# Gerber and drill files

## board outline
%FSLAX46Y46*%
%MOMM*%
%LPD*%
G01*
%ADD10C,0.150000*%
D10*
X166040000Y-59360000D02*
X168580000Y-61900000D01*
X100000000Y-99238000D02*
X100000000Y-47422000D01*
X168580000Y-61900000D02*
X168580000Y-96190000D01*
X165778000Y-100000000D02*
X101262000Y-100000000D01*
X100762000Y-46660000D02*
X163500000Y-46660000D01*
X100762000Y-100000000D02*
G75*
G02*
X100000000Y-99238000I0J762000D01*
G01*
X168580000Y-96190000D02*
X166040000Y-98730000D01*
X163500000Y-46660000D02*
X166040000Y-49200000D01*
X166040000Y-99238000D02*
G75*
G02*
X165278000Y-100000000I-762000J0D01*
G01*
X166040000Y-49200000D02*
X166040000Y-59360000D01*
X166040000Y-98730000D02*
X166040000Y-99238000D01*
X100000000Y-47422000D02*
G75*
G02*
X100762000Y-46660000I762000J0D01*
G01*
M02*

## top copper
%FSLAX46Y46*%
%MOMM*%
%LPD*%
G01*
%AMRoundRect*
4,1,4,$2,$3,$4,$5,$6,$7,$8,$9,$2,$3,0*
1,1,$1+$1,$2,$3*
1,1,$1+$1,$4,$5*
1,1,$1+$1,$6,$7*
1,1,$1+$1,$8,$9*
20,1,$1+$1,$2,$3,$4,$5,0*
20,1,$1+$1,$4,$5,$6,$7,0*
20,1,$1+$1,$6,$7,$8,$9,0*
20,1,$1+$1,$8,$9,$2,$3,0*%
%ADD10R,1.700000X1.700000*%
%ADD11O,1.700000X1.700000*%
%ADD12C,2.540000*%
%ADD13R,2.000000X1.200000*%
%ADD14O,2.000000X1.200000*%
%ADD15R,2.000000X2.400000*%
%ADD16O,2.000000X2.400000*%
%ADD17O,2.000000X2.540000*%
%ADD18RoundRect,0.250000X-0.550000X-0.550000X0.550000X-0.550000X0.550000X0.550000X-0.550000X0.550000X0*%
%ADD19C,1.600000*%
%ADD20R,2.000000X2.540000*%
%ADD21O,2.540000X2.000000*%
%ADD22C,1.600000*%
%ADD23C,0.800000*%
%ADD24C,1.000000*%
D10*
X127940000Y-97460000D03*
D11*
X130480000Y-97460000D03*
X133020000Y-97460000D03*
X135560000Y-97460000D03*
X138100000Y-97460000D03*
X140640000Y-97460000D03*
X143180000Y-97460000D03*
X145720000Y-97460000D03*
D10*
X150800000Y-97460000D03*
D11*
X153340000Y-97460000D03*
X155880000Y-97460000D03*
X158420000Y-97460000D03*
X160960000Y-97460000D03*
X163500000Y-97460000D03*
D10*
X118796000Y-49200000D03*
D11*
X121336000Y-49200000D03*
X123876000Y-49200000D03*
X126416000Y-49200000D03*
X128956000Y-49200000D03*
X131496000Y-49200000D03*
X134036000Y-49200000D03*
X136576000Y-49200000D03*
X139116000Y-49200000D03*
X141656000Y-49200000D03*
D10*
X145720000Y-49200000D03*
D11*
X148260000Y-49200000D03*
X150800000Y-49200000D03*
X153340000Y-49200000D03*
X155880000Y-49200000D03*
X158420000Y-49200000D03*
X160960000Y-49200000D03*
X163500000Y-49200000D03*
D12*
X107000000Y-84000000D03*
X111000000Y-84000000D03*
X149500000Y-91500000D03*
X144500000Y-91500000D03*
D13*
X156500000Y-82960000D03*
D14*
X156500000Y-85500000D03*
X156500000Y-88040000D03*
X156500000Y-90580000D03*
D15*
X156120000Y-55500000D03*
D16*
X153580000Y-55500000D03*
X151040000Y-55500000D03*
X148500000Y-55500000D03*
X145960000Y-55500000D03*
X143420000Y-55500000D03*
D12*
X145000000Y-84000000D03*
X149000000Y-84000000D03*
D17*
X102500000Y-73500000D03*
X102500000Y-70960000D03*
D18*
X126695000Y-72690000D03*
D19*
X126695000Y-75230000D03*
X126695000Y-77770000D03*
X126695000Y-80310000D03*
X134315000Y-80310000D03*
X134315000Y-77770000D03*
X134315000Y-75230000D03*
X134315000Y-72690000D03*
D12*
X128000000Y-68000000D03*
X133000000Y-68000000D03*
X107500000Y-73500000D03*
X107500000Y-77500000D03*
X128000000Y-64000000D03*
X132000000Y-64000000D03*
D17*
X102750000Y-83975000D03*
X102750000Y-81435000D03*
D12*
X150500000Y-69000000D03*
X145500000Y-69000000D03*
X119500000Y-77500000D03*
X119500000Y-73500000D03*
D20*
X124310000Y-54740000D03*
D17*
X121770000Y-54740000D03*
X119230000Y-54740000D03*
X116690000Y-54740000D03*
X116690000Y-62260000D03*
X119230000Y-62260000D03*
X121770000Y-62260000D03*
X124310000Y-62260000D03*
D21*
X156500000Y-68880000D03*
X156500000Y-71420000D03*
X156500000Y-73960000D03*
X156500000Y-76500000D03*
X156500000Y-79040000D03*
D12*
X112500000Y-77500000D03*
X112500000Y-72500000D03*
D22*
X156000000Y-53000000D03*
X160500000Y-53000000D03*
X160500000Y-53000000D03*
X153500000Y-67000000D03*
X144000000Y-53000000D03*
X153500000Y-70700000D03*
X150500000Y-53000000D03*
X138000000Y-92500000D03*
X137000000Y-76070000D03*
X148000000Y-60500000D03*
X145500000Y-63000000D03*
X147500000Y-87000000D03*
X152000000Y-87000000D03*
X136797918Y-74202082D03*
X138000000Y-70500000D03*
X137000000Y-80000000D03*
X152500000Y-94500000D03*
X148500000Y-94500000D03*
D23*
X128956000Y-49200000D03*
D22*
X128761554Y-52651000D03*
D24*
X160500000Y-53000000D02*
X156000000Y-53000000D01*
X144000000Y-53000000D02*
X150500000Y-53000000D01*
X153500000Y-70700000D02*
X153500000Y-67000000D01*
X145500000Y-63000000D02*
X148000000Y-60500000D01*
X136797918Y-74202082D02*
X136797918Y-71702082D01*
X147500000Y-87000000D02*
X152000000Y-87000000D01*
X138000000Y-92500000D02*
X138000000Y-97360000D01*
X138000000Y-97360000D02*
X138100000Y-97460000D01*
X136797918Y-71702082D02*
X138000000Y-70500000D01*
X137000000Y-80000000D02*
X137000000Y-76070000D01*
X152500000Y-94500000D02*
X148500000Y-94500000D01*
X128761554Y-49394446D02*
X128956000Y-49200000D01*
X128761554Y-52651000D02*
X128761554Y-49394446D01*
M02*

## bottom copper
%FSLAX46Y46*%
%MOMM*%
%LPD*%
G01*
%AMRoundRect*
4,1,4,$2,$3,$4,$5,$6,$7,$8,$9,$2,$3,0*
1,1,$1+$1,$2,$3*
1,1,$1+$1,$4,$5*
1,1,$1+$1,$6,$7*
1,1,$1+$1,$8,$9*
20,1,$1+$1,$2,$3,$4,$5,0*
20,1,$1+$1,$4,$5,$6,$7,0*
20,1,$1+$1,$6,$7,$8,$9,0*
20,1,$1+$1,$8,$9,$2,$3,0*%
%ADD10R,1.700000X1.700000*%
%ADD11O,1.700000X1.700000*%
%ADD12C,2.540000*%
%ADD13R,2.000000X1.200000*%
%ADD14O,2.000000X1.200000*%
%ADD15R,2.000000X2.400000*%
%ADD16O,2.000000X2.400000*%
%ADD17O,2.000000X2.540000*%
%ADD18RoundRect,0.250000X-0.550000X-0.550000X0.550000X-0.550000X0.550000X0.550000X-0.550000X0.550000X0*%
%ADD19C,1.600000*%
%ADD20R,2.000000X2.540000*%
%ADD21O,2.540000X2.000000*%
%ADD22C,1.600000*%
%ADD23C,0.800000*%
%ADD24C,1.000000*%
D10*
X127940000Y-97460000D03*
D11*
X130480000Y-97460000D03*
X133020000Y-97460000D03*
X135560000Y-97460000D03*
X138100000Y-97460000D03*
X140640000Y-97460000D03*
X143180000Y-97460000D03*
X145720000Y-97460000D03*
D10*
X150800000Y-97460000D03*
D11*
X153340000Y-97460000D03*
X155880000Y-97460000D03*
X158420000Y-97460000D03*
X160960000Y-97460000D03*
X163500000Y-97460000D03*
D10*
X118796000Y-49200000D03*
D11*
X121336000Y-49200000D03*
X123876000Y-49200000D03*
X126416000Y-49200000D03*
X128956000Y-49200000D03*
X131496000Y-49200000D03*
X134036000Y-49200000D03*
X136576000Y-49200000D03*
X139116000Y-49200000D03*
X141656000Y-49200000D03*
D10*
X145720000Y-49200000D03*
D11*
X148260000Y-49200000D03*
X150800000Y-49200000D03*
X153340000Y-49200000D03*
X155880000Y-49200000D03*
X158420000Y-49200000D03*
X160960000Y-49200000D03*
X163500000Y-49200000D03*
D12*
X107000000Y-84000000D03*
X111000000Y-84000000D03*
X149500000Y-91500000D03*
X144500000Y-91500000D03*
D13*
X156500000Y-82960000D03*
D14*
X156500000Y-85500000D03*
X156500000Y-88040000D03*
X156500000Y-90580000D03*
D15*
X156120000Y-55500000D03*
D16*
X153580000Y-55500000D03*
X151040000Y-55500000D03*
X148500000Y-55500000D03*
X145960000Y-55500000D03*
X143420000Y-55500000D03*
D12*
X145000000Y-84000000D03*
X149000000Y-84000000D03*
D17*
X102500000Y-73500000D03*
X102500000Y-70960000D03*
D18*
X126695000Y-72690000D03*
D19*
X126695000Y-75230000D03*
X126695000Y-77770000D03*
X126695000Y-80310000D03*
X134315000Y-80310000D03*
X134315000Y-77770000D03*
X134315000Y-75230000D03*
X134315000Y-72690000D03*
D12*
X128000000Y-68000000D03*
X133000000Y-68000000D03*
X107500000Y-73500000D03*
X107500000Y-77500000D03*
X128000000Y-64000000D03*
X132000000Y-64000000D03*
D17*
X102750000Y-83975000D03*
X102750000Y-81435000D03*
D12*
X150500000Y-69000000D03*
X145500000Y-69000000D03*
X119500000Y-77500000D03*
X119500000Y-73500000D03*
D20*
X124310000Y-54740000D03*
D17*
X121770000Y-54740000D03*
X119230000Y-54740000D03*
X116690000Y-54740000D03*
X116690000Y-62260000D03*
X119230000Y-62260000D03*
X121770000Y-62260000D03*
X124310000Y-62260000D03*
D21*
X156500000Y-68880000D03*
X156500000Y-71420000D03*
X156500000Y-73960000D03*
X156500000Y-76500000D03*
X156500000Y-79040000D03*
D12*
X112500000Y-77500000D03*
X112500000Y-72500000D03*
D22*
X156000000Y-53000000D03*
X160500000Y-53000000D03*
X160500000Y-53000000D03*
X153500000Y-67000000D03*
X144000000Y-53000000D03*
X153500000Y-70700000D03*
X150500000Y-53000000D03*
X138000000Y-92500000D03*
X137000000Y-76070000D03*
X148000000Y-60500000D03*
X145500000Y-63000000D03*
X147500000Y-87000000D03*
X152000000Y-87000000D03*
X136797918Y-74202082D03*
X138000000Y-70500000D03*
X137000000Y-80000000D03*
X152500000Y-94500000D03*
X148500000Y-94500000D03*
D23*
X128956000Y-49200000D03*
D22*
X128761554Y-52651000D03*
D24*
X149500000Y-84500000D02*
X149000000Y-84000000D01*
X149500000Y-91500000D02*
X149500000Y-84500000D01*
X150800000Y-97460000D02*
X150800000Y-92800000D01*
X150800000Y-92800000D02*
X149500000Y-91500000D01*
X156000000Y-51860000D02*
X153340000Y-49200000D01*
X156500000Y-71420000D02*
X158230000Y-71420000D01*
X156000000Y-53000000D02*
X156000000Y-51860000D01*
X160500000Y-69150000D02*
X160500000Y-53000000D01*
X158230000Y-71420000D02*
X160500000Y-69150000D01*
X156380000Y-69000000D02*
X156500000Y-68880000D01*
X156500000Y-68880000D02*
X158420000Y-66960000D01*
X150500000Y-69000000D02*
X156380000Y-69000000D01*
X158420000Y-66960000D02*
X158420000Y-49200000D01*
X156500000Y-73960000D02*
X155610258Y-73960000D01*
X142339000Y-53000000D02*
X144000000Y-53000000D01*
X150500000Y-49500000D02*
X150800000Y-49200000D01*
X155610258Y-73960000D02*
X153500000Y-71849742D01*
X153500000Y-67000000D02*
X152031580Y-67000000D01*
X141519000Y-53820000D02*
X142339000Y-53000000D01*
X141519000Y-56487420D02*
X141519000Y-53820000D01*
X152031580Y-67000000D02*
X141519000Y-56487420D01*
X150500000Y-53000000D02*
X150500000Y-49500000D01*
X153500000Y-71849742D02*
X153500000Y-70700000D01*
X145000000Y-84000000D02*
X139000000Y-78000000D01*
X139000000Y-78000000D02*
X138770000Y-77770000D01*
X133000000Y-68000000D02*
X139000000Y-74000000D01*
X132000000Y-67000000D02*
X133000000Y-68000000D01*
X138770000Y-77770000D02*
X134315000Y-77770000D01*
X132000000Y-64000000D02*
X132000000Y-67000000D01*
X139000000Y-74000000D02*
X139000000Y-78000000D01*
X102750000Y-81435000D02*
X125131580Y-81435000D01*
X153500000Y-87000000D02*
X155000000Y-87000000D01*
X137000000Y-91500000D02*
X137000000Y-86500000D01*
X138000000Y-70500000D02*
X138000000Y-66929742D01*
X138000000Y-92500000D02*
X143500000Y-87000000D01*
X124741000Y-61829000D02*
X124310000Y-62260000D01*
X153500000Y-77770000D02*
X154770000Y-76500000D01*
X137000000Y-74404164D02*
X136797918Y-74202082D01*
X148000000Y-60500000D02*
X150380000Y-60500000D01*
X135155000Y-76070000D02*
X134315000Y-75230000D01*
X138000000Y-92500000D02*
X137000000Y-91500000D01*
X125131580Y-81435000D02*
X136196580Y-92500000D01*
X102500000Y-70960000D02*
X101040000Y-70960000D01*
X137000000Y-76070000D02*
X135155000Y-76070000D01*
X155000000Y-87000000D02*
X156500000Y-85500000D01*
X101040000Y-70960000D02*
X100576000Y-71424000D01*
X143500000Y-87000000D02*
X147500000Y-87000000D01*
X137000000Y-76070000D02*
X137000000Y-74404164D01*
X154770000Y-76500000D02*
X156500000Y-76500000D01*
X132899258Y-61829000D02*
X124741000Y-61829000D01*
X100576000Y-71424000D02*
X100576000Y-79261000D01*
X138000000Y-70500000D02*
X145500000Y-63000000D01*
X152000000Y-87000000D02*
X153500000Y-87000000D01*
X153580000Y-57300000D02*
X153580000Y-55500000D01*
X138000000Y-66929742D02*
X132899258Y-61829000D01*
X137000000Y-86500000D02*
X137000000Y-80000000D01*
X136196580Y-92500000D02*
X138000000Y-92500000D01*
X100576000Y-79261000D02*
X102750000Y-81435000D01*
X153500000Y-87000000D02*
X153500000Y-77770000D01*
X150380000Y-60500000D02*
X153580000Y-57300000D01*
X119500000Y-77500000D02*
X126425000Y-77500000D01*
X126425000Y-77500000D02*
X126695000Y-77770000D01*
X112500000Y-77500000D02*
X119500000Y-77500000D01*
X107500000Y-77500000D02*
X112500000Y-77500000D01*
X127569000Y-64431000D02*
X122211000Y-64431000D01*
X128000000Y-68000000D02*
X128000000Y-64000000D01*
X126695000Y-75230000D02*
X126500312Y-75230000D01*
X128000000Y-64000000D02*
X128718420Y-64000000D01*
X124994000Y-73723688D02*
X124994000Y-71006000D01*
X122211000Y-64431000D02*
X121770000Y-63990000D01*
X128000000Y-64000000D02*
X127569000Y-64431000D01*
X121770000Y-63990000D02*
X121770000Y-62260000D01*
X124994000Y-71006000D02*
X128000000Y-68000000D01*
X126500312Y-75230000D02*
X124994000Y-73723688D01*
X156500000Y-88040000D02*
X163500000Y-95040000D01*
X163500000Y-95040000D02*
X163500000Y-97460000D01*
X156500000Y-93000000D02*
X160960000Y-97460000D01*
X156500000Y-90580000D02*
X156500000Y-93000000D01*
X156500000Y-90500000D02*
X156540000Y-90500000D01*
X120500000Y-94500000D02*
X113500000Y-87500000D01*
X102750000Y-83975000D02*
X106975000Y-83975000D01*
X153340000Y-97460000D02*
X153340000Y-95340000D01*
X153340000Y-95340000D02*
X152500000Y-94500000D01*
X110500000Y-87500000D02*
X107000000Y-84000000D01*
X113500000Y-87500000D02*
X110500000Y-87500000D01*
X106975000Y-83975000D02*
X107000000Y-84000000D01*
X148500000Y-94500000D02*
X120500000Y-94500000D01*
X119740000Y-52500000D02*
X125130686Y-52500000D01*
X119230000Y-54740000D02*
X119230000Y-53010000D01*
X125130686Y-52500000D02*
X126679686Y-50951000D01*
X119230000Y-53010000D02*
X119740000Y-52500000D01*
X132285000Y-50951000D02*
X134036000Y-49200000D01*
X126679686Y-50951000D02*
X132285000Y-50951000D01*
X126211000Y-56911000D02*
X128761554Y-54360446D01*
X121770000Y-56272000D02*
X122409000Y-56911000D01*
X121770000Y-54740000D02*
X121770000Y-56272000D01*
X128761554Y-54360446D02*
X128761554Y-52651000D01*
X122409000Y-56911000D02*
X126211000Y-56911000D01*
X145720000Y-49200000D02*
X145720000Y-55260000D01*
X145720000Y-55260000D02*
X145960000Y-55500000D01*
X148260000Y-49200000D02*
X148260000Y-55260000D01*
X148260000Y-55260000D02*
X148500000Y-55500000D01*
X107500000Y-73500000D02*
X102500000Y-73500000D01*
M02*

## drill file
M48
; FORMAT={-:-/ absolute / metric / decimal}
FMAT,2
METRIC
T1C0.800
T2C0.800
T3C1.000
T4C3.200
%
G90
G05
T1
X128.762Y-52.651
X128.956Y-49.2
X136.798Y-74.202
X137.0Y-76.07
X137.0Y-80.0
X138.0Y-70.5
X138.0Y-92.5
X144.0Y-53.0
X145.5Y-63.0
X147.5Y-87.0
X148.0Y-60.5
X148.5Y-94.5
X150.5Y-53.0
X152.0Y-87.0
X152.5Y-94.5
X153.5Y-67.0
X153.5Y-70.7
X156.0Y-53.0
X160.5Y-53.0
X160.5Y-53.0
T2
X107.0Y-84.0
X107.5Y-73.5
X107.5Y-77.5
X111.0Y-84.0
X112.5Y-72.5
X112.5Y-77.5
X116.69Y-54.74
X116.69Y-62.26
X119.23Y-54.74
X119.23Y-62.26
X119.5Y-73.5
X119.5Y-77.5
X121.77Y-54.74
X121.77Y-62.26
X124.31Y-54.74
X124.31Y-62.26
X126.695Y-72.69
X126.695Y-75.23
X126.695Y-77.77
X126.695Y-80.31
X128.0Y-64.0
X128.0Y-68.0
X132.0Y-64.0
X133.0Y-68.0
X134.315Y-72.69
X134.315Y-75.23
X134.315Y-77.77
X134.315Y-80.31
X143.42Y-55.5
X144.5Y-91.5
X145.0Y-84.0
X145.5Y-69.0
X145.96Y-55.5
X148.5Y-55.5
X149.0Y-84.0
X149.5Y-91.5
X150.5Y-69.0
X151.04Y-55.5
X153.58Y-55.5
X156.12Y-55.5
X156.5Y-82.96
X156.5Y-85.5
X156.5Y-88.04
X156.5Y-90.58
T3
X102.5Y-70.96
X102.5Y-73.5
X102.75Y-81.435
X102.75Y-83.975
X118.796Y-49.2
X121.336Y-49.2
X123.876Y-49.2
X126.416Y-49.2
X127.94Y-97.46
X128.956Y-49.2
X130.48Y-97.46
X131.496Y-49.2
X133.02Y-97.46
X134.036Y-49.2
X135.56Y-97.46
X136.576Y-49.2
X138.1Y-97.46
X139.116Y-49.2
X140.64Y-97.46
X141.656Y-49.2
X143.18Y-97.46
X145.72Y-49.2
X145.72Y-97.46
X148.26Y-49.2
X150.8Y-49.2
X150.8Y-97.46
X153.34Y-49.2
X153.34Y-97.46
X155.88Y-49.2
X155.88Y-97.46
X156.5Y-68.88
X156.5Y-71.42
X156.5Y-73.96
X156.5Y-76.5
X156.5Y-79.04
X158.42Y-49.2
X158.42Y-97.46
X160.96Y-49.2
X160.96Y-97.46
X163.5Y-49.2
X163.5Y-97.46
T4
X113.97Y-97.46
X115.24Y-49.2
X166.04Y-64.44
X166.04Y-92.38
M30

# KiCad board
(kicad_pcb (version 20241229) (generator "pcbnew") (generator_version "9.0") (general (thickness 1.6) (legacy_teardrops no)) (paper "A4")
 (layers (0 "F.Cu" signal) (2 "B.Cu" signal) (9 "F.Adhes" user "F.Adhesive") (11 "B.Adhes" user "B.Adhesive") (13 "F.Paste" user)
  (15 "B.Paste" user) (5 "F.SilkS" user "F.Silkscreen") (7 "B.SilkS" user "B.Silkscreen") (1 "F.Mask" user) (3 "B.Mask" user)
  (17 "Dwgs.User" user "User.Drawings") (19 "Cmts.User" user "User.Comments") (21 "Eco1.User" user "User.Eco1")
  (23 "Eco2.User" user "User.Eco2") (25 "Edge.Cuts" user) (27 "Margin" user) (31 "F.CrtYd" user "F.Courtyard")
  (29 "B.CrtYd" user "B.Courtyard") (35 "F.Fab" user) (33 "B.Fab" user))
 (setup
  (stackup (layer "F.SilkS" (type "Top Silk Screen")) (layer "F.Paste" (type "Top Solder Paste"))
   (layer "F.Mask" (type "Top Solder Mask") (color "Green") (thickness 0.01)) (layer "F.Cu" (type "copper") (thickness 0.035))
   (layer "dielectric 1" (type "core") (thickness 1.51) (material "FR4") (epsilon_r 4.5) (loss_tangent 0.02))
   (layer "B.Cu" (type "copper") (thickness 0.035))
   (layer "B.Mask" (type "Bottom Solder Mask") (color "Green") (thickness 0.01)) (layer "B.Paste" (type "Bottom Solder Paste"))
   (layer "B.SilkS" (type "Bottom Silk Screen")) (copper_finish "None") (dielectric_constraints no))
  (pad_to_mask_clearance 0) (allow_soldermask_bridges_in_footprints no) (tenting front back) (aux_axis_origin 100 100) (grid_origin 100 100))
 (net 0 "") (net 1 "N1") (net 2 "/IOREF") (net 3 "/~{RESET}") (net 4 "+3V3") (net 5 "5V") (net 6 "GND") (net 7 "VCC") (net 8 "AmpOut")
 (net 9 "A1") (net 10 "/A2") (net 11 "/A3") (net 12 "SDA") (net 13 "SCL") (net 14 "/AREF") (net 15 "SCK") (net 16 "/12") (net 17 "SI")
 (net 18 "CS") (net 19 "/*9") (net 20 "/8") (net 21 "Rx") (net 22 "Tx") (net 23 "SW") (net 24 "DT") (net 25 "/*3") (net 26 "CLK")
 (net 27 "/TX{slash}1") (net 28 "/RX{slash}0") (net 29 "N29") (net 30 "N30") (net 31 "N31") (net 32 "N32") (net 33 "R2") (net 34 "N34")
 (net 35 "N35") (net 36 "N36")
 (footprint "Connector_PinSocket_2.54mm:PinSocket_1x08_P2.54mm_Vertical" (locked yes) (layer "F.Cu") (at 127.94 97.46 90)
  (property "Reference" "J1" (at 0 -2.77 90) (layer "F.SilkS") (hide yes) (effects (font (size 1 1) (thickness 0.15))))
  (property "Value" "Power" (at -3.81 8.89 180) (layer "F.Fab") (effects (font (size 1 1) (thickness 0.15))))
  (pad "1" thru_hole rect (at 0 0 90) (size 1.7 1.7) (drill 1) (layers "*.Cu" "*.Mask") (remove_unused_layers no) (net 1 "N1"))
  (pad "2" thru_hole oval (at 0 2.54 90) (size 1.7 1.7) (drill 1) (layers "*.Cu" "*.Mask") (remove_unused_layers no) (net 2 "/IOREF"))
  (pad "3" thru_hole oval (at 0 5.08 90) (size 1.7 1.7) (drill 1) (layers "*.Cu" "*.Mask") (remove_unused_layers no) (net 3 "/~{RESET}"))
  (pad "4" thru_hole oval (at 0 7.62 90) (size 1.7 1.7) (drill 1) (layers "*.Cu" "*.Mask") (remove_unused_layers no) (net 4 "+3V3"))
  (pad "5" thru_hole oval (at 0 10.16 90) (size 1.7 1.7) (drill 1) (layers "*.Cu" "*.Mask") (remove_unused_layers no) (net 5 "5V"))
  (pad "6" thru_hole oval (at 0 12.7 90) (size 1.7 1.7) (drill 1) (layers "*.Cu" "*.Mask") (remove_unused_layers no) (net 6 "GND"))
  (pad "7" thru_hole oval (at 0 15.24 90) (size 1.7 1.7) (drill 1) (layers "*.Cu" "*.Mask") (remove_unused_layers no) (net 6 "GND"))
  (pad "8" thru_hole oval (at 0 17.78 90) (size 1.7 1.7) (drill 1) (layers "*.Cu" "*.Mask") (remove_unused_layers no) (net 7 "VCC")))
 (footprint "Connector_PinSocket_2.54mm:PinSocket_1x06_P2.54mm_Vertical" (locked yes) (layer "F.Cu") (at 150.8 97.46 90)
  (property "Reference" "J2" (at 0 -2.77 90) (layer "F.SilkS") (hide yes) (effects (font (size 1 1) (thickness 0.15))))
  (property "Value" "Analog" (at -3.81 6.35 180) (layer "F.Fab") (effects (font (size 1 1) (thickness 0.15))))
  (pad "1" thru_hole rect (at 0 0 90) (size 1.7 1.7) (drill 1) (layers "*.Cu" "*.Mask") (remove_unused_layers no) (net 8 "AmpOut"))
  (pad "2" thru_hole oval (at 0 2.54 90) (size 1.7 1.7) (drill 1) (layers "*.Cu" "*.Mask") (remove_unused_layers no) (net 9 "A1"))
  (pad "3" thru_hole oval (at 0 5.08 90) (size 1.7 1.7) (drill 1) (layers "*.Cu" "*.Mask") (remove_unused_layers no) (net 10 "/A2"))
  (pad "4" thru_hole oval (at 0 7.62 90) (size 1.7 1.7) (drill 1) (layers "*.Cu" "*.Mask") (remove_unused_layers no) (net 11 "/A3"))
  (pad "5" thru_hole oval (at 0 10.16 90) (size 1.7 1.7) (drill 1) (layers "*.Cu" "*.Mask") (remove_unused_layers no) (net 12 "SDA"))
  (pad "6" thru_hole oval (at 0 12.7 90) (size 1.7 1.7) (drill 1) (layers "*.Cu" "*.Mask") (remove_unused_layers no) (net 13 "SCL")))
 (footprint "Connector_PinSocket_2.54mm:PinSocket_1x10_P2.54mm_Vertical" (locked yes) (layer "F.Cu") (at 118.796 49.2 90)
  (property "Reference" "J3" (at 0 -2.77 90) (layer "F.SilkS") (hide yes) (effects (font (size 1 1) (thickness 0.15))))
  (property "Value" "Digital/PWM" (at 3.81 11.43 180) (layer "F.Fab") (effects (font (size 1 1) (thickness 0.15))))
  (pad "1" thru_hole rect (at 0 0 90) (size 1.7 1.7) (drill 1) (layers "*.Cu" "*.Mask") (remove_unused_layers no) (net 13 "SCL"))
  (pad "2" thru_hole oval (at 0 2.54 90) (size 1.7 1.7) (drill 1) (layers "*.Cu" "*.Mask") (remove_unused_layers no) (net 12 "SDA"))
  (pad "3" thru_hole oval (at 0 5.08 90) (size 1.7 1.7) (drill 1) (layers "*.Cu" "*.Mask") (remove_unused_layers no) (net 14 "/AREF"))
  (pad "4" thru_hole oval (at 0 7.62 90) (size 1.7 1.7) (drill 1) (layers "*.Cu" "*.Mask") (remove_unused_layers no) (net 6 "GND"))
  (pad "5" thru_hole oval (at 0 10.16 90) (size 1.7 1.7) (drill 1) (layers "*.Cu" "*.Mask") (remove_unused_layers no) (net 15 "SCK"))
  (pad "6" thru_hole oval (at 0 12.7 90) (size 1.7 1.7) (drill 1) (layers "*.Cu" "*.Mask") (remove_unused_layers no) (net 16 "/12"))
  (pad "7" thru_hole oval (at 0 15.24 90) (size 1.7 1.7) (drill 1) (layers "*.Cu" "*.Mask") (remove_unused_layers no) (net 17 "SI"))
  (pad "8" thru_hole oval (at 0 17.78 90) (size 1.7 1.7) (drill 1) (layers "*.Cu" "*.Mask") (remove_unused_layers no) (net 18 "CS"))
  (pad "9" thru_hole oval (at 0 20.32 90) (size 1.7 1.7) (drill 1) (layers "*.Cu" "*.Mask") (remove_unused_layers no) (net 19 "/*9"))
  (pad "10" thru_hole oval (at 0 22.86 90) (size 1.7 1.7) (drill 1) (layers "*.Cu" "*.Mask") (remove_unused_layers no) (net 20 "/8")))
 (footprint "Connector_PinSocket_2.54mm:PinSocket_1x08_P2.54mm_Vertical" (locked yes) (layer "F.Cu") (at 145.72 49.2 90)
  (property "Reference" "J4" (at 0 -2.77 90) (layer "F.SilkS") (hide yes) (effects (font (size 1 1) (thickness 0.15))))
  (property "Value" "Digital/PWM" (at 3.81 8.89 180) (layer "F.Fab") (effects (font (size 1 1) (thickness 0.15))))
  (pad "1" thru_hole rect (at 0 0 90) (size 1.7 1.7) (drill 1) (layers "*.Cu" "*.Mask") (remove_unused_layers no) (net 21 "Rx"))
  (pad "2" thru_hole oval (at 0 2.54 90) (size 1.7 1.7) (drill 1) (layers "*.Cu" "*.Mask") (remove_unused_layers no) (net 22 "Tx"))
  (pad "3" thru_hole oval (at 0 5.08 90) (size 1.7 1.7) (drill 1) (layers "*.Cu" "*.Mask") (remove_unused_layers no) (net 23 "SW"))
  (pad "4" thru_hole oval (at 0 7.62 90) (size 1.7 1.7) (drill 1) (layers "*.Cu" "*.Mask") (remove_unused_layers no) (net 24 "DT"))
  (pad "5" thru_hole oval (at 0 10.16 90) (size 1.7 1.7) (drill 1) (layers "*.Cu" "*.Mask") (remove_unused_layers no) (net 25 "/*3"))
  (pad "6" thru_hole oval (at 0 12.7 90) (size 1.7 1.7) (drill 1) (layers "*.Cu" "*.Mask") (remove_unused_layers no) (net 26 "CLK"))
  (pad "7" thru_hole oval (at 0 15.24 90) (size 1.7 1.7) (drill 1) (layers "*.Cu" "*.Mask") (remove_unused_layers no) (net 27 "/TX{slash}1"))
  (pad "8" thru_hole oval (at 0 17.78 90) (size 1.7 1.7) (drill 1) (layers "*.Cu" "*.Mask") (remove_unused_layers no) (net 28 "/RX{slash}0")))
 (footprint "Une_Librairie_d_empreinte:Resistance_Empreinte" (layer "F.Cu") (at 109 84)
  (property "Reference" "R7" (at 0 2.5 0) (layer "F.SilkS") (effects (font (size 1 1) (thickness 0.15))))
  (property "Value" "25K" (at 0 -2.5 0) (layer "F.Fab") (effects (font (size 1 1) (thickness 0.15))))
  (pad "1" thru_hole circle (at -2 0) (size 2.54 2.54) (drill 0.8) (layers "*.Cu" "*.Mask") (remove_unused_layers no) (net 9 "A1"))
  (pad "2" thru_hole circle (at 2 0) (size 2.54 2.54) (drill 0.8) (layers "*.Cu" "*.Mask") (remove_unused_layers no) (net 6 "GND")))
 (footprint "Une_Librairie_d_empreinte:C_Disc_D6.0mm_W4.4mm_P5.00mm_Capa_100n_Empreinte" (layer "F.Cu") (at 149.5 91.5 180)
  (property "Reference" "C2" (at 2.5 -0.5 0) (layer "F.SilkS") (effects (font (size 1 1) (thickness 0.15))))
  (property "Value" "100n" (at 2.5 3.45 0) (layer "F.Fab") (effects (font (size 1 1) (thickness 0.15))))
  (pad "1" thru_hole circle (at 0 0 180) (size 2.54 2.54) (drill 0.8) (layers "*.Cu" "*.Mask") (remove_unused_layers no) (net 8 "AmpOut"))
  (pad "2" thru_hole circle (at 5 0 180) (size 2.54 2.54) (drill 0.8) (layers "*.Cu" "*.Mask") (remove_unused_layers no) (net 6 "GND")))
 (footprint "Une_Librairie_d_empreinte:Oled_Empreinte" (layer "F.Cu") (at 156.5 86.77 -90)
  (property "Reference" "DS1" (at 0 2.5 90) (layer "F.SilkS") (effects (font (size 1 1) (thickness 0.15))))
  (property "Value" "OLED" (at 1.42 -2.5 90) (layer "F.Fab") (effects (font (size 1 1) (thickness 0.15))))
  (pad "1" thru_hole rect (at -3.81 0 270) (size 1.2 2) (drill 0.8) (layers "*.Cu" "*.Mask") (remove_unused_layers no) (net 6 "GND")
   (thermal_bridge_angle 45))
  (pad "2" thru_hole oval (at -1.27 0 270) (size 1.2 2) (drill 0.8) (layers "*.Cu" "*.Mask") (remove_unused_layers no) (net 5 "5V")
   (thermal_bridge_angle 45))
  (pad "3" thru_hole oval (at 1.27 0 270) (size 1.2 2) (drill 0.8) (layers "*.Cu" "*.Mask") (remove_unused_layers no) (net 13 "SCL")
   (thermal_bridge_angle 45))
  (pad "4" thru_hole oval (at 3.81 0 270) (size 1.2 2) (drill 0.8) (layers "*.Cu" "*.Mask") (remove_unused_layers no) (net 12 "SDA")
   (thermal_bridge_angle 45)))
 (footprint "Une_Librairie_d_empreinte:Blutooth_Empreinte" (layer "F.Cu") (at 149.77 55.5 180)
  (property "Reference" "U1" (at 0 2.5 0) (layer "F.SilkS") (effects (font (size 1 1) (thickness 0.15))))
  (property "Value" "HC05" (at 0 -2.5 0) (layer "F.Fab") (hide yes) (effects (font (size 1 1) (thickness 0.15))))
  (pad "1" thru_hole rect (at -6.35 0 180) (size 2 2.4) (drill 0.8) (layers "*.Cu" "*.Mask") (remove_unused_layers no) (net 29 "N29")
   (thermal_bridge_angle 45))
  (pad "2" thru_hole oval (at -3.81 0 180) (size 2 2.4) (drill 0.8) (layers "*.Cu" "*.Mask") (remove_unused_layers no) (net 5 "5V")
   (thermal_bridge_angle 45))
  (pad "3" thru_hole oval (at -1.27 0 180) (size 2 2.4) (drill 0.8) (layers "*.Cu" "*.Mask") (remove_unused_layers no) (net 6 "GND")
   (thermal_bridge_angle 45))
  (pad "4" thru_hole oval (at 1.27 0 180) (size 2 2.4) (drill 0.8) (layers "*.Cu" "*.Mask") (remove_unused_layers no) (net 22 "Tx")
   (thermal_bridge_angle 45))
  (pad "5" thru_hole oval (at 3.81 0 180) (size 2 2.4) (drill 0.8) (layers "*.Cu" "*.Mask") (remove_unused_layers no) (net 21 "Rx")
   (thermal_bridge_angle 45))
  (pad "6" thru_hole oval (at 6.35 0 180) (size 2 2.4) (drill 0.8) (layers "*.Cu" "*.Mask") (remove_unused_layers no) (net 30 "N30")
   (thermal_bridge_angle 45)))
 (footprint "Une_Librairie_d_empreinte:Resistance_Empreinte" (layer "F.Cu") (at 147 84)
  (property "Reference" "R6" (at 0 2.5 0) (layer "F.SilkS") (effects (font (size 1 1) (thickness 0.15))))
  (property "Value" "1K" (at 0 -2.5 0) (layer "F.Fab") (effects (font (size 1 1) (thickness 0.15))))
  (pad "1" thru_hole circle (at -2 0) (size 2.54 2.54) (drill 0.8) (layers "*.Cu" "*.Mask") (remove_unused_layers no) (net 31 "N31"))
  (pad "2" thru_hole circle (at 2 0) (size 2.54 2.54) (drill 0.8) (layers "*.Cu" "*.Mask") (remove_unused_layers no) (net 8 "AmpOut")))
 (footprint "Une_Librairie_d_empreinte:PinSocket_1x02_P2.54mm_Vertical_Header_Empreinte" (layer "F.Cu") (at 102.5 73.5 180)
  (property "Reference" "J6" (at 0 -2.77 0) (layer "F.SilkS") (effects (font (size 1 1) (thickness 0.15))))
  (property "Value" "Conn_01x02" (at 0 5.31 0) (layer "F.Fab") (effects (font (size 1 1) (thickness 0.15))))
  (pad "1" thru_hole oval (at 0 0 180) (size 2 2.54) (drill 1) (layers "*.Cu" "*.Mask") (remove_unused_layers no) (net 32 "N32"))
  (pad "2" thru_hole oval (at 0 2.54 180) (size 2 2.54) (drill 1) (layers "*.Cu" "*.Mask") (remove_unused_layers no) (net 5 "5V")))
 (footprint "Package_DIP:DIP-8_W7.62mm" (layer "F.Cu") (at 126.695 72.69)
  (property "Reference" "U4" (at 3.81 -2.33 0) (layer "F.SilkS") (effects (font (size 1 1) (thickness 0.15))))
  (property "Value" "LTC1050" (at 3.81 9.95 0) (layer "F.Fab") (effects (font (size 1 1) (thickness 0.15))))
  (pad "1" thru_hole roundrect (at 0 0) (size 1.6 1.6) (drill 0.8) (layers "*.Cu" "*.Mask") (remove_unused_layers no)
   (roundrect_rratio 0.15625))
  (pad "2" thru_hole circle (at 0 2.54) (size 1.6 1.6) (drill 0.8) (layers "*.Cu" "*.Mask") (remove_unused_layers no) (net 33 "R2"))
  (pad "3" thru_hole circle (at 0 5.08) (size 1.6 1.6) (drill 0.8) (layers "*.Cu" "*.Mask") (remove_unused_layers no) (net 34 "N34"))
  (pad "4" thru_hole circle (at 0 7.62) (size 1.6 1.6) (drill 0.8) (layers "*.Cu" "*.Mask") (remove_unused_layers no) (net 6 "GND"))
  (pad "5" thru_hole circle (at 7.62 7.62) (size 1.6 1.6) (drill 0.8) (layers "*.Cu" "*.Mask") (remove_unused_layers no) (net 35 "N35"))
  (pad "6" thru_hole circle (at 7.62 5.08) (size 1.6 1.6) (drill 0.8) (layers "*.Cu" "*.Mask") (remove_unused_layers no) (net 31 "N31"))
  (pad "7" thru_hole circle (at 7.62 2.54) (size 1.6 1.6) (drill 0.8) (layers "*.Cu" "*.Mask") (remove_unused_layers no) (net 5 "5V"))
  (pad "8" thru_hole circle (at 7.62 0) (size 1.6 1.6) (drill 0.8) (layers "*.Cu" "*.Mask") (remove_unused_layers no) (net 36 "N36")))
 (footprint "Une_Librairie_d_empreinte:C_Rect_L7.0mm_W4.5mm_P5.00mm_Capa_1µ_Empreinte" (layer "F.Cu") (at 128 68)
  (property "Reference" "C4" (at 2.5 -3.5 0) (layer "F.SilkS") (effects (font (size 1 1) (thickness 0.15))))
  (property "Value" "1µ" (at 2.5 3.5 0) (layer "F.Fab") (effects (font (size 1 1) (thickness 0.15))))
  (pad "1" thru_hole circle (at 0 0) (size 2.54 2.54) (drill 0.8) (layers "*.Cu" "*.Mask") (remove_unused_layers no) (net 33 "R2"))
  (pad "2" thru_hole circle (at 5 0) (size 2.54 2.54) (drill 0.8) (layers "*.Cu" "*.Mask") (remove_unused_layers no) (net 31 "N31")))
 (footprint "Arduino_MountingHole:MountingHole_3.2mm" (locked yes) (layer "F.Cu") (at 115.24 49.2)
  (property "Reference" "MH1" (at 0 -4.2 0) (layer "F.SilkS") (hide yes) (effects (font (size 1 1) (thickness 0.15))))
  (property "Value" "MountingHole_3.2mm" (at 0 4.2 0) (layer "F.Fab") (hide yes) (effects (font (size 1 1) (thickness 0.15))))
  (pad "" np_thru_hole circle (at 0 0) (size 3.2 3.2) (drill 3.2) (layers "*.Cu" "*.Mask")))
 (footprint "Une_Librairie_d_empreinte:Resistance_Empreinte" (layer "F.Cu") (at 107.5 75.5 -90)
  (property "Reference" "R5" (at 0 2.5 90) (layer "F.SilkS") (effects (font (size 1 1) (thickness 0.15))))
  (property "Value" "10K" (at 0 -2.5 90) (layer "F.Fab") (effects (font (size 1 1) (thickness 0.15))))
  (pad "1" thru_hole circle (at -2 0 270) (size 2.54 2.54) (drill 0.8) (layers "*.Cu" "*.Mask") (remove_unused_layers no) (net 32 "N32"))
  (pad "2" thru_hole circle (at 2 0 270) (size 2.54 2.54) (drill 0.8) (layers "*.Cu" "*.Mask") (remove_unused_layers no) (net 34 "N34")))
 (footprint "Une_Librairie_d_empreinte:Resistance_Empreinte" (layer "F.Cu") (at 130 64)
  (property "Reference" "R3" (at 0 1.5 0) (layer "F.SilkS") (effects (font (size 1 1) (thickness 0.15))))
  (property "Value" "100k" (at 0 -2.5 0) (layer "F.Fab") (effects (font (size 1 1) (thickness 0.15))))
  (pad "1" thru_hole circle (at -2 0) (size 2.54 2.54) (drill 0.8) (layers "*.Cu" "*.Mask") (remove_unused_layers no) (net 33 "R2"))
  (pad "2" thru_hole circle (at 2 0) (size 2.54 2.54) (drill 0.8) (layers "*.Cu" "*.Mask") (remove_unused_layers no) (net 31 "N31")))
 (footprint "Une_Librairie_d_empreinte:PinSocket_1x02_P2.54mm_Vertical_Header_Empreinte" (layer "F.Cu") (at 102.75 83.975 180)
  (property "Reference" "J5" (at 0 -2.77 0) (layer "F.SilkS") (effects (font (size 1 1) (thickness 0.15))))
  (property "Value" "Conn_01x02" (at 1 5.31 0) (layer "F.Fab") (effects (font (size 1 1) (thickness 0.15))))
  (pad "1" thru_hole oval (at 0 0 180) (size 2 2.54) (drill 1) (layers "*.Cu" "*.Mask") (remove_unused_layers no) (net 9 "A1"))
  (pad "2" thru_hole oval (at 0 2.54 180) (size 2 2.54) (drill 1) (layers "*.Cu" "*.Mask") (remove_unused_layers no) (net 5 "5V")))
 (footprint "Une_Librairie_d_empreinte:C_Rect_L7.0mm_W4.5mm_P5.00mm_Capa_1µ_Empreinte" (layer "F.Cu") (at 150.5 69 180)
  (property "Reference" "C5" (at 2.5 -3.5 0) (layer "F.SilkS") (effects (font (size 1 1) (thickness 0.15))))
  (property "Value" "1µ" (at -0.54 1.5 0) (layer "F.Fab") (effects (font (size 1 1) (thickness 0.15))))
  (pad "1" thru_hole circle (at 0 0 180) (size 2.54 2.54) (drill 0.8) (layers "*.Cu" "*.Mask") (remove_unused_layers no) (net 26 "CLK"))
  (pad "2" thru_hole circle (at 5 0 180) (size 2.54 2.54) (drill 0.8) (layers "*.Cu" "*.Mask") (remove_unused_layers no) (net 6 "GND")))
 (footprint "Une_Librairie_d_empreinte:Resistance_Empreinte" (layer "F.Cu") (at 119.5 75.5 90)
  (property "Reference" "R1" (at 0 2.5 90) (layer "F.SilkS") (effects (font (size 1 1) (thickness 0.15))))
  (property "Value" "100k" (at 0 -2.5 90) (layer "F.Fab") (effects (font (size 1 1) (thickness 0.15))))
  (pad "1" thru_hole circle (at -2 0 90) (size 2.54 2.54) (drill 0.8) (layers "*.Cu" "*.Mask") (remove_unused_layers no) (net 34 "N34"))
  (pad "2" thru_hole circle (at 2 0 90) (size 2.54 2.54) (drill 0.8) (layers "*.Cu" "*.Mask") (remove_unused_layers no) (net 6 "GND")))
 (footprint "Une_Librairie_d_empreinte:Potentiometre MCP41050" (layer "F.Cu") (at 120.5 58.5 180)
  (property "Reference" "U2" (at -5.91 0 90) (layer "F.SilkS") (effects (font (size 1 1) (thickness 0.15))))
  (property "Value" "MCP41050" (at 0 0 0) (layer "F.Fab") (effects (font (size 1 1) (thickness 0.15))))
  (pad "1" thru_hole rect (at -3.81 3.76 180) (size 2 2.54) (drill 0.8) (layers "*.Cu" "*.Mask") (remove_unused_layers no) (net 18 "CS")
   (thermal_bridge_angle 45))
  (pad "2" thru_hole oval (at -1.27 3.76 180) (size 2 2.54) (drill 0.8) (layers "*.Cu" "*.Mask") (remove_unused_layers no) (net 15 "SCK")
   (thermal_bridge_angle 45))
  (pad "3" thru_hole oval (at 1.27 3.76 180) (size 2 2.54) (drill 0.8) (layers "*.Cu" "*.Mask") (remove_unused_layers no) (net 17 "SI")
   (thermal_bridge_angle 45))
  (pad "4" thru_hole oval (at 3.81 3.76 180) (size 2 2.54) (drill 0.8) (layers "*.Cu" "*.Mask") (remove_unused_layers no) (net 6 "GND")
   (thermal_bridge_angle 45))
  (pad "5" thru_hole oval (at 3.81 -3.76 180) (size 2 2.54) (drill 0.8) (layers "*.Cu" "*.Mask") (remove_unused_layers no) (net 6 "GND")
   (thermal_bridge_angle 45))
  (pad "6" thru_hole oval (at 1.27 -3.76 180) (size 2 2.54) (drill 0.8) (layers "*.Cu" "*.Mask") (remove_unused_layers no) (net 6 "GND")
   (thermal_bridge_angle 45))
  (pad "7" thru_hole oval (at -1.27 -3.76 180) (size 2 2.54) (drill 0.8) (layers "*.Cu" "*.Mask") (remove_unused_layers no) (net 33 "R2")
   (thermal_bridge_angle 45))
  (pad "8" thru_hole oval (at -3.81 -3.76 180) (size 2 2.54) (drill 0.8) (layers "*.Cu" "*.Mask") (remove_unused_layers no) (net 5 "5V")
   (thermal_bridge_angle 45)))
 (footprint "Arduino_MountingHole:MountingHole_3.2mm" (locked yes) (layer "F.Cu") (at 113.97 97.46)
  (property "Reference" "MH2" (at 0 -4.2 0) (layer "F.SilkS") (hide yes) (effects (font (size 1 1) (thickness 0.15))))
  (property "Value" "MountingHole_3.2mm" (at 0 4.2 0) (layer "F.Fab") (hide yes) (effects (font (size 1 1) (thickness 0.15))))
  (pad "" np_thru_hole circle (at 0 0) (size 3.2 3.2) (drill 3.2) (layers "*.Cu" "*.Mask")))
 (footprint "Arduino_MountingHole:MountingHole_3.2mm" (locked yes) (layer "F.Cu") (at 166.04 64.44)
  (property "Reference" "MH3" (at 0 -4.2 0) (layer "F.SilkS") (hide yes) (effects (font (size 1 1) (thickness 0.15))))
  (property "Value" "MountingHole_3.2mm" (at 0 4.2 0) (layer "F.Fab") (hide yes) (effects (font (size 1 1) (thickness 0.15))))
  (pad "" np_thru_hole circle (at 0 0) (size 3.2 3.2) (drill 3.2) (layers "*.Cu" "*.Mask")))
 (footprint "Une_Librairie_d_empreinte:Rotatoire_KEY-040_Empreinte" (layer "F.Cu") (at 156.5 73.96 -90)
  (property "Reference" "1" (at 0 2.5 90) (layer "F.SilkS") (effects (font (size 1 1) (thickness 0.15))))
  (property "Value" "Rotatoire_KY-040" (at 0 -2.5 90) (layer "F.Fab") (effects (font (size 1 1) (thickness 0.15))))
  (pad "1" thru_hole oval (at -5.08 0 270) (size 2 2.54) (drill 1) (layers "*.Cu" "*.Mask") (remove_unused_layers no) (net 26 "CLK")
   (thermal_bridge_angle 45))
  (pad "2" thru_hole oval (at -2.54 0 270) (size 2 2.54) (drill 1) (layers "*.Cu" "*.Mask") (remove_unused_layers no) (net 24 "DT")
   (thermal_bridge_angle 45))
  (pad "3" thru_hole oval (at 0 0 270) (size 2 2.54) (drill 1) (layers "*.Cu" "*.Mask") (remove_unused_layers no) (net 23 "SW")
   (thermal_bridge_angle 45))
  (pad "4" thru_hole oval (at 2.54 0 270) (size 2 2.54) (drill 1) (layers "*.Cu" "*.Mask") (remove_unused_layers no) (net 5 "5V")
   (thermal_bridge_angle 45))
  (pad "5" thru_hole oval (at 5.08 0 270) (size 2 2.54) (drill 1) (layers "*.Cu" "*.Mask") (remove_unused_layers no) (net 6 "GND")
   (thermal_bridge_angle 45)))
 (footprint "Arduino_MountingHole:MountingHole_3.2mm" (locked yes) (layer "F.Cu") (at 166.04 92.38)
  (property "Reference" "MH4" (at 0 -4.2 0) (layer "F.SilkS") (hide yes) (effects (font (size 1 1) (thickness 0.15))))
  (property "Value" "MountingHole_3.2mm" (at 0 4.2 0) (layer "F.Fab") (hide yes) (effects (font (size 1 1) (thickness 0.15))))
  (pad "" np_thru_hole circle (at 0 0) (size 3.2 3.2) (drill 3.2) (layers "*.Cu" "*.Mask")))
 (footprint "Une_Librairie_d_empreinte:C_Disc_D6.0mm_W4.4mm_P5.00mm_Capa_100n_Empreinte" (layer "F.Cu") (at 112.5 77.5 90)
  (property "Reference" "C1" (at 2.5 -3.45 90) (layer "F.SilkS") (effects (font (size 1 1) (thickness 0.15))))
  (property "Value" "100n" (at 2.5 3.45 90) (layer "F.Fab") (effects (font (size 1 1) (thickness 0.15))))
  (pad "1" thru_hole circle (at 0 0 90) (size 2.54 2.54) (drill 0.8) (layers "*.Cu" "*.Mask") (remove_unused_layers no) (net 34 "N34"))
  (pad "2" thru_hole circle (at 5 0 90) (size 2.54 2.54) (drill 0.8) (layers "*.Cu" "*.Mask") (remove_unused_layers no) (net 6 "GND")))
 (gr_line (start 166.04 59.36) (end 168.58 61.9) (stroke (width 0.15) (type solid)) (layer "Edge.Cuts"))
 (gr_line (start 100 99.238) (end 100 47.422) (stroke (width 0.15) (type solid)) (layer "Edge.Cuts"))
 (gr_line (start 168.58 61.9) (end 168.58 96.19) (stroke (width 0.15) (type solid)) (layer "Edge.Cuts"))
 (gr_line (start 165.778 100) (end 101.262 100) (stroke (width 0.15) (type solid)) (layer "Edge.Cuts"))
 (gr_line (start 100.762 46.66) (end 163.5 46.66) (stroke (width 0.15) (type solid)) (layer "Edge.Cuts"))
 (gr_arc (start 100.762 100) (mid 100.223185 99.776815) (end 100 99.238) (stroke (width 0.15) (type solid)) (layer "Edge.Cuts"))
 (gr_line (start 168.58 96.19) (end 166.04 98.73) (stroke (width 0.15) (type solid)) (layer "Edge.Cuts"))
 (gr_line (start 163.5 46.66) (end 166.04 49.2) (stroke (width 0.15) (type solid)) (layer "Edge.Cuts"))
 (gr_arc (start 166.04 99.238) (mid 165.816815 99.776815) (end 165.278 100) (stroke (width 0.15) (type solid)) (layer "Edge.Cuts"))
 (gr_line (start 166.04 49.2) (end 166.04 59.36) (stroke (width 0.15) (type solid)) (layer "Edge.Cuts"))
 (gr_line (start 166.04 98.73) (end 166.04 99.238) (stroke (width 0.15) (type solid)) (layer "Edge.Cuts"))
 (gr_arc (start 100 47.422) (mid 100.223185 46.883185) (end 100.762 46.66) (stroke (width 0.15) (type solid)) (layer "Edge.Cuts"))
 (segment (start 149.5 84.5) (end 149 84) (width 1) (layer "B.Cu") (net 8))
 (segment (start 149.5 91.5) (end 149.5 84.5) (width 1) (layer "B.Cu") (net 8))
 (segment (start 150.8 97.46) (end 150.8 92.8) (width 1) (layer "B.Cu") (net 8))
 (segment (start 150.8 92.8) (end 149.5 91.5) (width 1) (layer "B.Cu") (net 8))
 (segment (start 160.5 53) (end 156 53) (width 1) (layer "F.Cu") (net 24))
 (via (at 156 53) (size 1.6) (drill 0.8) (layers "F.Cu" "B.Cu") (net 24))
 (via (at 160.5 53) (size 1.6) (drill 0.8) (layers "F.Cu" "B.Cu") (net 24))
 (via (at 160.5 53) (size 1.6) (drill 0.8) (layers "F.Cu" "B.Cu") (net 24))
 (segment (start 156 51.86) (end 153.34 49.2) (width 1) (layer "B.Cu") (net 24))
 (segment (start 156.5 71.42) (end 158.23 71.42) (width 1) (layer "B.Cu") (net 24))
 (segment (start 156 53) (end 156 51.86) (width 1) (layer "B.Cu") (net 24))
 (segment (start 160.5 69.15) (end 160.5 53) (width 1) (layer "B.Cu") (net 24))
 (segment (start 158.23 71.42) (end 160.5 69.15) (width 1) (layer "B.Cu") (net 24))
 (segment (start 156.38 69) (end 156.5 68.88) (width 1) (layer "B.Cu") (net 26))
 (segment (start 156.5 68.88) (end 158.42 66.96) (width 1) (layer "B.Cu") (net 26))
 (segment (start 150.5 69) (end 156.38 69) (width 1) (layer "B.Cu") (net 26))
 (segment (start 158.42 66.96) (end 158.42 49.2) (width 1) (layer "B.Cu") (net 26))
 (segment (start 144 53) (end 150.5 53) (width 1) (layer "F.Cu") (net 23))
 (segment (start 153.5 70.7) (end 153.5 67) (width 1) (layer "F.Cu") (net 23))
 (via (at 153.5 67) (size 1.6) (drill 0.8) (layers "F.Cu" "B.Cu") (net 23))
 (via (at 144 53) (size 1.6) (drill 0.8) (layers "F.Cu" "B.Cu") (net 23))
 (via (at 153.5 70.7) (size 1.6) (drill 0.8) (layers "F.Cu" "B.Cu") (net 23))
 (via (at 150.5 53) (size 1.6) (drill 0.8) (layers "F.Cu" "B.Cu") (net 23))
 (segment (start 156.5 73.96) (end 155.610258 73.96) (width 1) (layer "B.Cu") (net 23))
 (segment (start 142.339 53) (end 144 53) (width 1) (layer "B.Cu") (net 23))
 (segment (start 150.5 49.5) (end 150.8 49.2) (width 1) (layer "B.Cu") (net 23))
 (segment (start 155.610258 73.96) (end 153.5 71.849742) (width 1) (layer "B.Cu") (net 23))
 (segment (start 153.5 67) (end 152.03158 67) (width 1) (layer "B.Cu") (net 23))
 (segment (start 141.519 53.82) (end 142.339 53) (width 1) (layer "B.Cu") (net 23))
 (segment (start 141.519 56.48742) (end 141.519 53.82) (width 1) (layer "B.Cu") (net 23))
 (segment (start 152.03158 67) (end 141.519 56.48742) (width 1) (layer "B.Cu") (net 23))
 (segment (start 150.5 53) (end 150.5 49.5) (width 1) (layer "B.Cu") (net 23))
 (segment (start 153.5 71.849742) (end 153.5 70.7) (width 1) (layer "B.Cu") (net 23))
 (segment (start 145 84) (end 139 78) (width 1) (layer "B.Cu") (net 31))
 (segment (start 139 78) (end 138.77 77.77) (width 1) (layer "B.Cu") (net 31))
 (segment (start 133 68) (end 139 74) (width 1) (layer "B.Cu") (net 31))
 (segment (start 132 67) (end 133 68) (width 1) (layer "B.Cu") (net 31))
 (segment (start 138.77 77.77) (end 134.315 77.77) (width 1) (layer "B.Cu") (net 31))
 (segment (start 132 64) (end 132 67) (width 1) (layer "B.Cu") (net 31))
 (segment (start 139 74) (end 139 78) (width 1) (layer "B.Cu") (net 31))
 (segment (start 145.5 63) (end 148 60.5) (width 1) (layer "F.Cu") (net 5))
 (segment (start 136.797918 74.202082) (end 136.797918 71.702082) (width 1) (layer "F.Cu") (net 5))
 (segment (start 147.5 87) (end 152 87) (width 1) (layer "F.Cu") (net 5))
 (segment (start 138 92.5) (end 138 97.36) (width 1) (layer "F.Cu") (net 5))
 (segment (start 138 97.36) (end 138.1 97.46) (width 1) (layer "F.Cu") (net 5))
 (segment (start 136.797918 71.702082) (end 138 70.5) (width 1) (layer "F.Cu") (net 5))
 (segment (start 137 80) (end 137 76.07) (width 1) (layer "F.Cu") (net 5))
 (via (at 138 92.5) (size 1.6) (drill 0.8) (layers "F.Cu" "B.Cu") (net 5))
 (via (at 137 76.07) (size 1.6) (drill 0.8) (layers "F.Cu" "B.Cu") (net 5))
 (via (at 148 60.5) (size 1.6) (drill 0.8) (layers "F.Cu" "B.Cu") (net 5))
 (via (at 145.5 63) (size 1.6) (drill 0.8) (layers "F.Cu" "B.Cu") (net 5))
 (via (at 147.5 87) (size 1.6) (drill 0.8) (layers "F.Cu" "B.Cu") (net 5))
 (via (at 152 87) (size 1.6) (drill 0.8) (layers "F.Cu" "B.Cu") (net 5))
 (via (at 136.797918 74.202082) (size 1.6) (drill 0.8) (layers "F.Cu" "B.Cu") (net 5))
 (via (at 138 70.5) (size 1.6) (drill 0.8) (layers "F.Cu" "B.Cu") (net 5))
 (via (at 137 80) (size 1.6) (drill 0.8) (layers "F.Cu" "B.Cu") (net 5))
 (segment (start 102.75 81.435) (end 125.13158 81.435) (width 1) (layer "B.Cu") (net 5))
 (segment (start 153.5 87) (end 155 87) (width 1) (layer "B.Cu") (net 5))
 (segment (start 137 91.5) (end 137 86.5) (width 1) (layer "B.Cu") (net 5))
 (segment (start 138 70.5) (end 138 66.929742) (width 1) (layer "B.Cu") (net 5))
 (segment (start 138 92.5) (end 143.5 87) (width 1) (layer "B.Cu") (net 5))
 (segment (start 124.741 61.829) (end 124.31 62.26) (width 1) (layer "B.Cu") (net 5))
 (segment (start 153.5 77.77) (end 154.77 76.5) (width 1) (layer "B.Cu") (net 5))
 (segment (start 137 74.404164) (end 136.797918 74.202082) (width 1) (layer "B.Cu") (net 5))
 (segment (start 148 60.5) (end 150.38 60.5) (width 1) (layer "B.Cu") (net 5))
 (segment (start 135.155 76.07) (end 134.315 75.23) (width 1) (layer "B.Cu") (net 5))
 (segment (start 138 92.5) (end 137 91.5) (width 1) (layer "B.Cu") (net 5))
 (segment (start 125.13158 81.435) (end 136.19658 92.5) (width 1) (layer "B.Cu") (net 5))
 (segment (start 102.5 70.96) (end 101.04 70.96) (width 1) (layer "B.Cu") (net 5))
 (segment (start 137 76.07) (end 135.155 76.07) (width 1) (layer "B.Cu") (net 5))
 (segment (start 155 87) (end 156.5 85.5) (width 1) (layer "B.Cu") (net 5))
 (segment (start 101.04 70.96) (end 100.576 71.424) (width 1) (layer "B.Cu") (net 5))
 (segment (start 143.5 87) (end 147.5 87) (width 1) (layer "B.Cu") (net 5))
 (segment (start 137 76.07) (end 137 74.404164) (width 1) (layer "B.Cu") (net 5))
 (segment (start 154.77 76.5) (end 156.5 76.5) (width 1) (layer "B.Cu") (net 5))
 (segment (start 132.899258 61.829) (end 124.741 61.829) (width 1) (layer "B.Cu") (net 5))
 (segment (start 100.576 71.424) (end 100.576 79.261) (width 1) (layer "B.Cu") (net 5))
 (segment (start 138 70.5) (end 145.5 63) (width 1) (layer "B.Cu") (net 5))
 (segment (start 152 87) (end 153.5 87) (width 1) (layer "B.Cu") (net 5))
 (segment (start 153.58 57.3) (end 153.58 55.5) (width 1) (layer "B.Cu") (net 5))
 (segment (start 138 66.929742) (end 132.899258 61.829) (width 1) (layer "B.Cu") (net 5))
 (segment (start 137 86.5) (end 137 80) (width 1) (layer "B.Cu") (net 5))
 (segment (start 136.19658 92.5) (end 138 92.5) (width 1) (layer "B.Cu") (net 5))
 (segment (start 100.576 79.261) (end 102.75 81.435) (width 1) (layer "B.Cu") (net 5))
 (segment (start 153.5 87) (end 153.5 77.77) (width 1) (layer "B.Cu") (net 5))
 (segment (start 150.38 60.5) (end 153.58 57.3) (width 1) (layer "B.Cu") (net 5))
 (segment (start 119.5 77.5) (end 126.425 77.5) (width 1) (layer "B.Cu") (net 34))
 (segment (start 126.425 77.5) (end 126.695 77.77) (width 1) (layer "B.Cu") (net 34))
 (segment (start 112.5 77.5) (end 119.5 77.5) (width 1) (layer "B.Cu") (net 34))
 (segment (start 107.5 77.5) (end 112.5 77.5) (width 1) (layer "B.Cu") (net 34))
 (segment (start 127.569 64.431) (end 122.211 64.431) (width 1) (layer "B.Cu") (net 33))
 (segment (start 128 68) (end 128 64) (width 1) (layer "B.Cu") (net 33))
 (segment (start 126.695 75.23) (end 126.500312 75.23) (width 1) (layer "B.Cu") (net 33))
 (segment (start 128 64) (end 128.71842 64) (width 1) (layer "B.Cu") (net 33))
 (segment (start 124.994 73.723688) (end 124.994 71.006) (width 1) (layer "B.Cu") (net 33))
 (segment (start 122.211 64.431) (end 121.77 63.99) (width 1) (layer "B.Cu") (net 33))
 (segment (start 128 64) (end 127.569 64.431) (width 1) (layer "B.Cu") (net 33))
 (segment (start 121.77 63.99) (end 121.77 62.26) (width 1) (layer "B.Cu") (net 33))
 (segment (start 124.994 71.006) (end 128 68) (width 1) (layer "B.Cu") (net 33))
 (segment (start 126.500312 75.23) (end 124.994 73.723688) (width 1) (layer "B.Cu") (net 33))
 (segment (start 156.5 88.04) (end 163.5 95.04) (width 1) (layer "B.Cu") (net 13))
 (segment (start 163.5 95.04) (end 163.5 97.46) (width 1) (layer "B.Cu") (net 13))
 (segment (start 156.5 93) (end 160.96 97.46) (width 1) (layer "B.Cu") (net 12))
 (segment (start 156.5 90.58) (end 156.5 93) (width 1) (layer "B.Cu") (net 12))
 (segment (start 156.5 90.5) (end 156.54 90.5) (width 1) (layer "B.Cu") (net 12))
 (segment (start 152.5 94.5) (end 148.5 94.5) (width 1) (layer "F.Cu") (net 9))
 (via (at 152.5 94.5) (size 1.6) (drill 0.8) (layers "F.Cu" "B.Cu") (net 9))
 (via (at 148.5 94.5) (size 1.6) (drill 0.8) (layers "F.Cu" "B.Cu") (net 9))
 (segment (start 120.5 94.5) (end 113.5 87.5) (width 1) (layer "B.Cu") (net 9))
 (segment (start 102.75 83.975) (end 106.975 83.975) (width 1) (layer "B.Cu") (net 9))
 (segment (start 153.34 97.46) (end 153.34 95.34) (width 1) (layer "B.Cu") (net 9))
 (segment (start 153.34 95.34) (end 152.5 94.5) (width 1) (layer "B.Cu") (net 9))
 (segment (start 110.5 87.5) (end 107 84) (width 1) (layer "B.Cu") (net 9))
 (segment (start 113.5 87.5) (end 110.5 87.5) (width 1) (layer "B.Cu") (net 9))
 (segment (start 106.975 83.975) (end 107 84) (width 1) (layer "B.Cu") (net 9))
 (segment (start 148.5 94.5) (end 120.5 94.5) (width 1) (layer "B.Cu") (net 9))
 (segment (start 119.74 52.5) (end 125.130686 52.5) (width 1) (layer "B.Cu") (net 17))
 (segment (start 119.23 54.74) (end 119.23 53.01) (width 1) (layer "B.Cu") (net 17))
 (segment (start 125.130686 52.5) (end 126.679686 50.951) (width 1) (layer "B.Cu") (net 17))
 (segment (start 119.23 53.01) (end 119.74 52.5) (width 1) (layer "B.Cu") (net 17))
 (segment (start 132.285 50.951) (end 134.036 49.2) (width 1) (layer "B.Cu") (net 17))
 (segment (start 126.679686 50.951) (end 132.285 50.951) (width 1) (layer "B.Cu") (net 17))
 (segment (start 128.761554 49.394446) (end 128.956 49.2) (width 1) (layer "F.Cu") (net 15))
 (segment (start 128.761554 52.651) (end 128.761554 49.394446) (width 1) (layer "F.Cu") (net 15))
 (via micro (at 128.956 49.2) (size 0.8) (drill 0.8) (layers "F.Cu" "B.Cu") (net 15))
 (via (at 128.761554 52.651) (size 1.6) (drill 0.8) (layers "F.Cu" "B.Cu") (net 15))
 (segment (start 126.211 56.911) (end 128.761554 54.360446) (width 1) (layer "B.Cu") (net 15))
 (segment (start 121.77 56.272) (end 122.409 56.911) (width 1) (layer "B.Cu") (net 15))
 (segment (start 121.77 54.74) (end 121.77 56.272) (width 1) (layer "B.Cu") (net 15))
 (segment (start 128.761554 54.360446) (end 128.761554 52.651) (width 1) (layer "B.Cu") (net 15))
 (segment (start 122.409 56.911) (end 126.211 56.911) (width 1) (layer "B.Cu") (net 15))
 (segment (start 145.72 49.2) (end 145.72 55.26) (width 1) (layer "B.Cu") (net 21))
 (segment (start 145.72 55.26) (end 145.96 55.5) (width 1) (layer "B.Cu") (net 21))
 (segment (start 148.26 49.2) (end 148.26 55.26) (width 1) (layer "B.Cu") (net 22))
 (segment (start 148.26 55.26) (end 148.5 55.5) (width 1) (layer "B.Cu") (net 22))
 (segment (start 107.5 73.5) (end 102.5 73.5) (width 1) (layer "B.Cu") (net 32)))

